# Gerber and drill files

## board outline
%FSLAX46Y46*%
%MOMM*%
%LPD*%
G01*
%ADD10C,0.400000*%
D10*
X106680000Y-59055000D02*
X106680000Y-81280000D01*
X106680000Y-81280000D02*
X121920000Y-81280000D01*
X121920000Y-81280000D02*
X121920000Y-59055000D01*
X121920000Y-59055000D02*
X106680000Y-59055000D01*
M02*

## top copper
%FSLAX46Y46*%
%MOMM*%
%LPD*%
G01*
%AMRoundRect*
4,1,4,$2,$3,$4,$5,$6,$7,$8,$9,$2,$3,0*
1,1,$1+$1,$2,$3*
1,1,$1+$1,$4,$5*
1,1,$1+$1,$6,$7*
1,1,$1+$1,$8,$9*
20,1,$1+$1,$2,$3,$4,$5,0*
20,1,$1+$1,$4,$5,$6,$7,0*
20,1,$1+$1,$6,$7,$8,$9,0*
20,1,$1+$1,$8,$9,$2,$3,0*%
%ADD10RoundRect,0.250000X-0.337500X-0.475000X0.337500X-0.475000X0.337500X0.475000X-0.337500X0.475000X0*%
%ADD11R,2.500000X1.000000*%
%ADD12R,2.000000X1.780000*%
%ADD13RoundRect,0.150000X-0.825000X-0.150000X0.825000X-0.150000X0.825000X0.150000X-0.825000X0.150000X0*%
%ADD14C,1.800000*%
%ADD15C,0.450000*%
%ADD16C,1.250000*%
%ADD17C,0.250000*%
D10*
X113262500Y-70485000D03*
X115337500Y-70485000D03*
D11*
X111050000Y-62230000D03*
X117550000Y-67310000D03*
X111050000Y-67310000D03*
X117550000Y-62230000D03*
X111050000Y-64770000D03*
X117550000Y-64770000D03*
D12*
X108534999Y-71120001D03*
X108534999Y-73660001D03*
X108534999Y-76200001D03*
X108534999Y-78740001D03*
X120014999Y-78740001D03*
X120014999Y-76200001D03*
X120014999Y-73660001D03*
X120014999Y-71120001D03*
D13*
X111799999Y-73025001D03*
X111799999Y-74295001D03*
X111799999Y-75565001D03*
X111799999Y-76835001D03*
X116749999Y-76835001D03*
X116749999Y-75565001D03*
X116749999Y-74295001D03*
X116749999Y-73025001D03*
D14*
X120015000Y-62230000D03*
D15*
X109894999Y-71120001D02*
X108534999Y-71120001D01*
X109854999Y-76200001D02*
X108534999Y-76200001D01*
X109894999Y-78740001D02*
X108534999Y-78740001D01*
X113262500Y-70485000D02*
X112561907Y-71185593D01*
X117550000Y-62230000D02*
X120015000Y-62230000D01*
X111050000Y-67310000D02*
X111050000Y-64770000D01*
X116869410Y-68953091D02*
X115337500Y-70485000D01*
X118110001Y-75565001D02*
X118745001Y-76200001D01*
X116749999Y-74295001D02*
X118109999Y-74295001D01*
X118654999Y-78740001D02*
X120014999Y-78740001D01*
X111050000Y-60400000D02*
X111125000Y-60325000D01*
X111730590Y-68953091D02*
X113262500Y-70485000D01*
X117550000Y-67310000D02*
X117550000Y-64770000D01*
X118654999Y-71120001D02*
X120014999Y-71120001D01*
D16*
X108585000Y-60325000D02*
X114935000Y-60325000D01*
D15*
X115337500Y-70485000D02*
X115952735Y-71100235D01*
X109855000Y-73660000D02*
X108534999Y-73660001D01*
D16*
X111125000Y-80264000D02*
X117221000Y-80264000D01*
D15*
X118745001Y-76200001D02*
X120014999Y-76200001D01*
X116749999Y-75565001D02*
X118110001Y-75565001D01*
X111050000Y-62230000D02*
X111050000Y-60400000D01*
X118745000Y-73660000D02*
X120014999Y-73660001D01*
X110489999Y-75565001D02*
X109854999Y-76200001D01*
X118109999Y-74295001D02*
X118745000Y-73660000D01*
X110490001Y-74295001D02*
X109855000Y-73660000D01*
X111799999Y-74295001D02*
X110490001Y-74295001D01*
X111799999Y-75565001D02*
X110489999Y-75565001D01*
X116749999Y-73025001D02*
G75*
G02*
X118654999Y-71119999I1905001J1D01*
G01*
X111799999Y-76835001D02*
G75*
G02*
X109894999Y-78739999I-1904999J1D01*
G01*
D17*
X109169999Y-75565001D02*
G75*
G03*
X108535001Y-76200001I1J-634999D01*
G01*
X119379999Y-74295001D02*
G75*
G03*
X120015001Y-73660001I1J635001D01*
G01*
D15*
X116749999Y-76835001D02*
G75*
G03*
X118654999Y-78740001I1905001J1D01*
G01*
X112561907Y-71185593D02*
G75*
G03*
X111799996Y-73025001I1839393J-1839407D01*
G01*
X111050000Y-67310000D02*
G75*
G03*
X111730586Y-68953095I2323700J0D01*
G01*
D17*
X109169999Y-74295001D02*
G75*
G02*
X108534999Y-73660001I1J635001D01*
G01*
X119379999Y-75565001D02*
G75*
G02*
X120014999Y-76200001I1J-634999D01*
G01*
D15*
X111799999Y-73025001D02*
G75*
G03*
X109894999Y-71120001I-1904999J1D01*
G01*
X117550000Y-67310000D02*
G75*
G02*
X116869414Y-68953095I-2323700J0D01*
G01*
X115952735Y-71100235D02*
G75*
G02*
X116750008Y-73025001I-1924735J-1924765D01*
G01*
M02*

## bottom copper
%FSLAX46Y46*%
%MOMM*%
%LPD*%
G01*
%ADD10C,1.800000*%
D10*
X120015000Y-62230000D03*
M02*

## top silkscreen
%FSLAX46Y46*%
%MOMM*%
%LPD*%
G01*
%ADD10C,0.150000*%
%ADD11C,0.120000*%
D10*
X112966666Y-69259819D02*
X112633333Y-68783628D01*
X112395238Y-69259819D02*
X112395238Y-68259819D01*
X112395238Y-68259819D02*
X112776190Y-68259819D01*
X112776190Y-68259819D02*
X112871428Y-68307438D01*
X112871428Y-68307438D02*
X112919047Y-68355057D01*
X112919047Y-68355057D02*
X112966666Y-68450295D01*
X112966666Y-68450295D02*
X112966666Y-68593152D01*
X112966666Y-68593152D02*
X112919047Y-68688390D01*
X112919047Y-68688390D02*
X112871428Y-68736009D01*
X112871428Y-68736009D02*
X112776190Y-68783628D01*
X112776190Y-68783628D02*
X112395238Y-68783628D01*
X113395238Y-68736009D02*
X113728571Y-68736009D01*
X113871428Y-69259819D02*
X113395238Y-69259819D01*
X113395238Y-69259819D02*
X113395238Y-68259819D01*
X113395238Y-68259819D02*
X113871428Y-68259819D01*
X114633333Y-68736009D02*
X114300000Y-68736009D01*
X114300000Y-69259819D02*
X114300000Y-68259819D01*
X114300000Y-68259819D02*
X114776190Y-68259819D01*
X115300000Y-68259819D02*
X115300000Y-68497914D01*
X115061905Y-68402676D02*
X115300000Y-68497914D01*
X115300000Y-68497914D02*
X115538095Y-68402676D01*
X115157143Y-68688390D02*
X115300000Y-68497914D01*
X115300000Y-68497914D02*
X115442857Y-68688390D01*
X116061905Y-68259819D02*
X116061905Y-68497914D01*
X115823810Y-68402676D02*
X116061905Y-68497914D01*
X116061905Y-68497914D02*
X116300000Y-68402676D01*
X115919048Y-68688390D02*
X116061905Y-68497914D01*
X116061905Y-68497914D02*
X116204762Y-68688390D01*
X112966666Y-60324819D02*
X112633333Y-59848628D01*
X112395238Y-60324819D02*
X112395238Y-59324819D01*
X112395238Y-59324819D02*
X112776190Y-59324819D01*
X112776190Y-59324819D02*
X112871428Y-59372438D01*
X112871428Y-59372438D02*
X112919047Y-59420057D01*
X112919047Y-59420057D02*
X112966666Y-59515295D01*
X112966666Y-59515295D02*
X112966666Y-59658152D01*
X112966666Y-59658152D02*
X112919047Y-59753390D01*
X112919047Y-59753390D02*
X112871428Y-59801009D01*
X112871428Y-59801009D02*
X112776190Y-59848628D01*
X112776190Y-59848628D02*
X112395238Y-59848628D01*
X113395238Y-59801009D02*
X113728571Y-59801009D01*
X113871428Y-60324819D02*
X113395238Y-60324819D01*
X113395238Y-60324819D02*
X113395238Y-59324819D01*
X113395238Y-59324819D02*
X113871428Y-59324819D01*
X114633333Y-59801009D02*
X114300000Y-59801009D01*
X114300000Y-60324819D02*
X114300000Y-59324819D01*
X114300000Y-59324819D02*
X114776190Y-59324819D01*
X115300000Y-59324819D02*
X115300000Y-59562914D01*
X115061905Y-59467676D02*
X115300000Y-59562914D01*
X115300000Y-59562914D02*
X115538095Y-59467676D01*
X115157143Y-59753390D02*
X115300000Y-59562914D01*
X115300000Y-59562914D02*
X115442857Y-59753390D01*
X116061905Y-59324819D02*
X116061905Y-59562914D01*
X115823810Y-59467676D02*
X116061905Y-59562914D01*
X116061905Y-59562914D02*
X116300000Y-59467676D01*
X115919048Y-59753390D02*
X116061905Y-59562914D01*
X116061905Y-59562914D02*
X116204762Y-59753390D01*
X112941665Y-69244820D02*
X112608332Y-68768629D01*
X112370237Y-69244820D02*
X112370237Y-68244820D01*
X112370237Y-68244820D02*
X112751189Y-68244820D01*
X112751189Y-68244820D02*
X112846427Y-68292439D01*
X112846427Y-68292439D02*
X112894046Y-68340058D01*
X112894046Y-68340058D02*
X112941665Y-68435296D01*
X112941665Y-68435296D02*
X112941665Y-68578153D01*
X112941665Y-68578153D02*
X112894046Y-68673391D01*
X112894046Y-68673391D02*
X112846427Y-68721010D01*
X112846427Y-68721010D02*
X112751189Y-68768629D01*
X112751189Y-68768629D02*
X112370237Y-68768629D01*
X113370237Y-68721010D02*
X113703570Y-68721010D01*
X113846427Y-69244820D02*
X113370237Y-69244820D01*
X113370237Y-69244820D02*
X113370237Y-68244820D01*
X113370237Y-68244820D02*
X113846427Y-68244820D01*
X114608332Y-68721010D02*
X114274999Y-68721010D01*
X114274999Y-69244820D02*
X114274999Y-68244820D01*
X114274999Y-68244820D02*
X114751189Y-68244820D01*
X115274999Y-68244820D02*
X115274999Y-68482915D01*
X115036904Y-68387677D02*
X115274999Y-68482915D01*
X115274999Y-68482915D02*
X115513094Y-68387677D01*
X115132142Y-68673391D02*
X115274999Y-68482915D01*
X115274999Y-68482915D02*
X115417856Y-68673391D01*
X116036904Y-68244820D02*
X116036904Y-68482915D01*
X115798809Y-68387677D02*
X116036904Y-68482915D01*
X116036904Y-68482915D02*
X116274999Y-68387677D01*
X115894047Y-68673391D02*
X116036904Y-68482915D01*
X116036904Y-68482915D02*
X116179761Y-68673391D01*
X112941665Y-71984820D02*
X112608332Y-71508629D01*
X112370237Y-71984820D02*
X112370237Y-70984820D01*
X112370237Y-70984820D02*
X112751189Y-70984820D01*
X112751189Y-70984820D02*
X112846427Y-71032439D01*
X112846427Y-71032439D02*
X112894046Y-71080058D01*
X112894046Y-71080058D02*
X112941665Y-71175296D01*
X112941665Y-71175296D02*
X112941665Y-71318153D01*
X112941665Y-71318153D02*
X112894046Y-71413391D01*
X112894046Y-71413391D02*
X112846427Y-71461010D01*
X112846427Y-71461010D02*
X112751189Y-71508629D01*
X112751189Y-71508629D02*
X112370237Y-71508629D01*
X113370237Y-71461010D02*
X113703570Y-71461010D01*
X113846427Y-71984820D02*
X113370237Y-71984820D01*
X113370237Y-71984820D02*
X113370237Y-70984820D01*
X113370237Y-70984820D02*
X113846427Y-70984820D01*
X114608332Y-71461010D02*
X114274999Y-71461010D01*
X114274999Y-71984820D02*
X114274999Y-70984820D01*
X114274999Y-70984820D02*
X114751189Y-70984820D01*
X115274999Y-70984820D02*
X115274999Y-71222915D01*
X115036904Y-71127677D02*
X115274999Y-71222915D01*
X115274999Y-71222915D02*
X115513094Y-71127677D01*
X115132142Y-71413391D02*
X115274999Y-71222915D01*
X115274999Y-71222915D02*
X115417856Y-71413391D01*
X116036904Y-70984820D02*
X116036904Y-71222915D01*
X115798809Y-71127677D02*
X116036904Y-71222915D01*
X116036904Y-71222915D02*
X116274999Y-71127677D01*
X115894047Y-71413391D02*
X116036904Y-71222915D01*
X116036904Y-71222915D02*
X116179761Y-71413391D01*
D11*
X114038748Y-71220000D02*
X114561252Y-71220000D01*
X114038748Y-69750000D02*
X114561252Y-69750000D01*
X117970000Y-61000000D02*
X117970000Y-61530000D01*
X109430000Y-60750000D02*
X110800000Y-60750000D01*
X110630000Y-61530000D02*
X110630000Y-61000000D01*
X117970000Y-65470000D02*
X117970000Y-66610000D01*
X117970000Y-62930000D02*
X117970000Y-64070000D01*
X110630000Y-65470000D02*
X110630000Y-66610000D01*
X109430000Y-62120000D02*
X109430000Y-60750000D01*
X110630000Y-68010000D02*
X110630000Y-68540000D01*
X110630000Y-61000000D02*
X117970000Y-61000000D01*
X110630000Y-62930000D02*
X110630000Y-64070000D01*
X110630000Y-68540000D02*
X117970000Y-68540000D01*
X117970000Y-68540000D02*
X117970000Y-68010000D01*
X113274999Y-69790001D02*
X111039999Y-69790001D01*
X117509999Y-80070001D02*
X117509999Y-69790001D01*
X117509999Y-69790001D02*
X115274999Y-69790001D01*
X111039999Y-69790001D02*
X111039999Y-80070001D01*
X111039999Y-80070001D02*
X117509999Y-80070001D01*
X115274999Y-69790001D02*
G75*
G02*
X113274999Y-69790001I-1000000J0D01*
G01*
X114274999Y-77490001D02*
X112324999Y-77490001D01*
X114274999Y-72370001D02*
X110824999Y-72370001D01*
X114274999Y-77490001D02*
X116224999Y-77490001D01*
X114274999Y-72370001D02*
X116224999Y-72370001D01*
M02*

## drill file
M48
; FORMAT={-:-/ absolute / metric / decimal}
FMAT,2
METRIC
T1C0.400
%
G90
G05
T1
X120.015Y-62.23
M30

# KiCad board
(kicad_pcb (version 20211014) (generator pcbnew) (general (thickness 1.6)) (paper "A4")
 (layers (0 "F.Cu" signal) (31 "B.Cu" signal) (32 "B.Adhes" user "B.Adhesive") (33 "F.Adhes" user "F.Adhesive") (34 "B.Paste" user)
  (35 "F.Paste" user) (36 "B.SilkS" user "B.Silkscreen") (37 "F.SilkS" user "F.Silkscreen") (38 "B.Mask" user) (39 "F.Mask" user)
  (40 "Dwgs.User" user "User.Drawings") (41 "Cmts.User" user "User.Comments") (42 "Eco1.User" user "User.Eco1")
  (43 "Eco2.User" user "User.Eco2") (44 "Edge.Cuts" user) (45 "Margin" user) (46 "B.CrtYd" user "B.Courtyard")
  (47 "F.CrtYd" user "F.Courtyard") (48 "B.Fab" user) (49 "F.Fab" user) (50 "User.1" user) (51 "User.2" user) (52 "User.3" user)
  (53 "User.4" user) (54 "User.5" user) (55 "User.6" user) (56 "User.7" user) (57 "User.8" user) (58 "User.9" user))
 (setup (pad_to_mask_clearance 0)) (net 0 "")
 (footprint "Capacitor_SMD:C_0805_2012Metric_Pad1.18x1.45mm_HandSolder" (layer "F.Cu") (at 114.3 70.485)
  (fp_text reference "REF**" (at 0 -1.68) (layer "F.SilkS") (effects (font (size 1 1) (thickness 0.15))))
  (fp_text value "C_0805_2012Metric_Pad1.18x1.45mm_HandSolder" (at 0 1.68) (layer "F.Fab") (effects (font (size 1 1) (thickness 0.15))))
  (fp_line (start -0.261252 0.735) (end 0.261252 0.735) (layer "F.SilkS") (width 0.12))
  (fp_line (start -0.261252 -0.735) (end 0.261252 -0.735) (layer "F.SilkS") (width 0.12))
  (pad "1" smd roundrect (at -1.0375 0) (size 1.175 1.45) (layers "F.Cu" "F.Paste" "F.Mask") (roundrect_rratio 0.2127659574))
  (pad "2" smd roundrect (at 1.0375 0) (size 1.175 1.45) (layers "F.Cu" "F.Paste" "F.Mask") (roundrect_rratio 0.2127659574)))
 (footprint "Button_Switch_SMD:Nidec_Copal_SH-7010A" (layer "F.Cu") (at 114.3 64.77)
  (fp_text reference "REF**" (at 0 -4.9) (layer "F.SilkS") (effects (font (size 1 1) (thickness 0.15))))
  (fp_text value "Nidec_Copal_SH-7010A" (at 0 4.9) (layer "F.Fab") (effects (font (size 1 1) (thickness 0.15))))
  (fp_line (start 3.67 -3.77) (end 3.67 -3.24) (layer "F.SilkS") (width 0.12))
  (fp_line (start -4.87 -4.02) (end -3.5 -4.02) (layer "F.SilkS") (width 0.12))
  (fp_line (start -3.67 -3.24) (end -3.67 -3.77) (layer "F.SilkS") (width 0.12))
  (fp_line (start 3.67 0.7) (end 3.67 1.84) (layer "F.SilkS") (width 0.12))
  (fp_line (start 3.67 -1.84) (end 3.67 -0.7) (layer "F.SilkS") (width 0.12))
  (fp_line (start -3.67 0.7) (end -3.67 1.84) (layer "F.SilkS") (width 0.12))
  (fp_line (start -4.87 -2.65) (end -4.87 -4.02) (layer "F.SilkS") (width 0.12))
  (fp_line (start -3.67 3.24) (end -3.67 3.77) (layer "F.SilkS") (width 0.12))
  (fp_line (start -3.67 -3.77) (end 3.67 -3.77) (layer "F.SilkS") (width 0.12))
  (fp_line (start -3.67 -1.84) (end -3.67 -0.7) (layer "F.SilkS") (width 0.12))
  (fp_line (start -3.67 3.77) (end 3.67 3.77) (layer "F.SilkS") (width 0.12))
  (fp_line (start 3.67 3.77) (end 3.67 3.24) (layer "F.SilkS") (width 0.12))
  (pad "1" smd rect (at -3.25 -2.54) (size 2.5 1) (layers "F.Cu" "F.Paste" "F.Mask"))
  (pad "2" smd rect (at 3.25 2.54) (size 2.5 1) (layers "F.Cu" "F.Paste" "F.Mask"))
  (pad "4" smd rect (at -3.25 2.54) (size 2.5 1) (layers "F.Cu" "F.Paste" "F.Mask"))
  (pad "8" smd rect (at 3.25 -2.54) (size 2.5 1) (layers "F.Cu" "F.Paste" "F.Mask"))
  (pad "C" smd rect (at -3.25 0) (size 2.5 1) (layers "F.Cu" "F.Paste" "F.Mask"))
  (pad "C" smd rect (at 3.25 0) (size 2.5 1) (layers "F.Cu" "F.Paste" "F.Mask")))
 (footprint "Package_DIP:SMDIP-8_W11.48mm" (layer "F.Cu") (at 114.274999 74.930001)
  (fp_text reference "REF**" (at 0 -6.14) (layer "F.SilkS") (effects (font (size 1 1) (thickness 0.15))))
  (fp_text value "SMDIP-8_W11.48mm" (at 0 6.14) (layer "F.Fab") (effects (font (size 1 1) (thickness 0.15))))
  (fp_line (start -1 -5.14) (end -3.235 -5.14) (layer "F.SilkS") (width 0.12))
  (fp_line (start 3.235 5.14) (end 3.235 -5.14) (layer "F.SilkS") (width 0.12))
  (fp_line (start 3.235 -5.14) (end 1 -5.14) (layer "F.SilkS") (width 0.12))
  (fp_line (start -3.235 -5.14) (end -3.235 5.14) (layer "F.SilkS") (width 0.12))
  (fp_line (start -3.235 5.14) (end 3.235 5.14) (layer "F.SilkS") (width 0.12))
  (fp_arc (start 1 -5.14) (mid 0 -4.14) (end -1 -5.14) (layer "F.SilkS") (width 0.12))
  (pad "1" smd rect (at -5.74 -3.81) (size 2 1.78) (layers "F.Cu" "F.Paste" "F.Mask"))
  (pad "2" smd rect (at -5.74 -1.27) (size 2 1.78) (layers "F.Cu" "F.Paste" "F.Mask"))
  (pad "3" smd rect (at -5.74 1.27) (size 2 1.78) (layers "F.Cu" "F.Paste" "F.Mask"))
  (pad "4" smd rect (at -5.74 3.81) (size 2 1.78) (layers "F.Cu" "F.Paste" "F.Mask"))
  (pad "5" smd rect (at 5.74 3.81) (size 2 1.78) (layers "F.Cu" "F.Paste" "F.Mask"))
  (pad "6" smd rect (at 5.74 1.27) (size 2 1.78) (layers "F.Cu" "F.Paste" "F.Mask"))
  (pad "7" smd rect (at 5.74 -1.27) (size 2 1.78) (layers "F.Cu" "F.Paste" "F.Mask"))
  (pad "8" smd rect (at 5.74 -3.81) (size 2 1.78) (layers "F.Cu" "F.Paste" "F.Mask")))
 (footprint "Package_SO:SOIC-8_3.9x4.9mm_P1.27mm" (layer "F.Cu") (at 114.274999 74.930001)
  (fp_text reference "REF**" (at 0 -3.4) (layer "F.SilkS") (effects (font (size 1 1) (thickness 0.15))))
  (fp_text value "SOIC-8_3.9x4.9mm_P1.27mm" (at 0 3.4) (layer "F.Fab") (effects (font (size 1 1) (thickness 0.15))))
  (fp_line (start 0 2.56) (end -1.95 2.56) (layer "F.SilkS") (width 0.12))
  (fp_line (start 0 -2.56) (end -3.45 -2.56) (layer "F.SilkS") (width 0.12))
  (fp_line (start 0 2.56) (end 1.95 2.56) (layer "F.SilkS") (width 0.12))
  (fp_line (start 0 -2.56) (end 1.95 -2.56) (layer "F.SilkS") (width 0.12))
  (pad "1" smd roundrect (at -2.475 -1.905) (size 1.95 0.6) (layers "F.Cu" "F.Paste" "F.Mask") (roundrect_rratio 0.25))
  (pad "2" smd roundrect (at -2.475 -0.635) (size 1.95 0.6) (layers "F.Cu" "F.Paste" "F.Mask") (roundrect_rratio 0.25))
  (pad "3" smd roundrect (at -2.475 0.635) (size 1.95 0.6) (layers "F.Cu" "F.Paste" "F.Mask") (roundrect_rratio 0.25))
  (pad "4" smd roundrect (at -2.475 1.905) (size 1.95 0.6) (layers "F.Cu" "F.Paste" "F.Mask") (roundrect_rratio 0.25))
  (pad "5" smd roundrect (at 2.475 1.905) (size 1.95 0.6) (layers "F.Cu" "F.Paste" "F.Mask") (roundrect_rratio 0.25))
  (pad "6" smd roundrect (at 2.475 0.635) (size 1.95 0.6) (layers "F.Cu" "F.Paste" "F.Mask") (roundrect_rratio 0.25))
  (pad "7" smd roundrect (at 2.475 -0.635) (size 1.95 0.6) (layers "F.Cu" "F.Paste" "F.Mask") (roundrect_rratio 0.25))
  (pad "8" smd roundrect (at 2.475 -1.905) (size 1.95 0.6) (layers "F.Cu" "F.Paste" "F.Mask") (roundrect_rratio 0.25)))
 (gr_line (start 106.68 59.055) (end 106.68 81.28) (layer "Edge.Cuts") (width 0.4))
 (gr_line (start 106.68 81.28) (end 121.92 81.28) (layer "Edge.Cuts") (width 0.4))
 (gr_line (start 121.92 81.28) (end 121.92 59.055) (layer "Edge.Cuts") (width 0.4))
 (gr_line (start 121.92 59.055) (end 106.68 59.055) (layer "Edge.Cuts") (width 0.4))
 (segment (start 109.894999 71.120001) (end 108.534999 71.120001) (width 0.45) (layer "F.Cu") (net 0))
 (segment (start 109.854999 76.200001) (end 108.534999 76.200001) (width 0.45) (layer "F.Cu") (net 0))
 (segment (start 109.894999 78.740001) (end 108.534999 78.740001) (width 0.45) (layer "F.Cu") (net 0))
 (segment (start 113.2625 70.485) (end 112.561907 71.185593) (width 0.45) (layer "F.Cu") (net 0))
 (segment (start 117.55 62.23) (end 120.015 62.23) (width 0.45) (layer "F.Cu") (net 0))
 (segment (start 111.05 67.31) (end 111.05 64.77) (width 0.45) (layer "F.Cu") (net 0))
 (segment (start 116.86941 68.953091) (end 115.3375 70.485) (width 0.45) (layer "F.Cu") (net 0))
 (segment (start 118.110001 75.565001) (end 118.745001 76.200001) (width 0.45) (layer "F.Cu") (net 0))
 (segment (start 116.749999 74.295001) (end 118.109999 74.295001) (width 0.45) (layer "F.Cu") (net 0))
 (segment (start 118.654999 78.740001) (end 120.014999 78.740001) (width 0.45) (layer "F.Cu") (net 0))
 (segment (start 111.05 60.4) (end 111.125 60.325) (width 0.45) (layer "F.Cu") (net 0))
 (segment (start 111.73059 68.953091) (end 113.2625 70.485) (width 0.45) (layer "F.Cu") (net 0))
 (segment (start 117.55 67.31) (end 117.55 64.77) (width 0.45) (layer "F.Cu") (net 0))
 (segment (start 118.654999 71.120001) (end 120.014999 71.120001) (width 0.45) (layer "F.Cu") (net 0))
 (segment (start 108.585 60.325) (end 114.935 60.325) (width 1.25) (layer "F.Cu") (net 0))
 (segment (start 115.3375 70.485) (end 115.952735 71.100235) (width 0.45) (layer "F.Cu") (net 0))
 (segment (start 109.855 73.66) (end 108.534999 73.660001) (width 0.45) (layer "F.Cu") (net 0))
 (segment (start 111.125 80.264) (end 117.221 80.264) (width 1.25) (layer "F.Cu") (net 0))
 (segment (start 118.745001 76.200001) (end 120.014999 76.200001) (width 0.45) (layer "F.Cu") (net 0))
 (segment (start 116.749999 75.565001) (end 118.110001 75.565001) (width 0.45) (layer "F.Cu") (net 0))
 (segment (start 111.05 62.23) (end 111.05 60.4) (width 0.45) (layer "F.Cu") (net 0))
 (segment (start 118.745 73.66) (end 120.014999 73.660001) (width 0.45) (layer "F.Cu") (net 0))
 (segment (start 110.489999 75.565001) (end 109.854999 76.200001) (width 0.45) (layer "F.Cu") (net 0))
 (segment (start 118.109999 74.295001) (end 118.745 73.66) (width 0.45) (layer "F.Cu") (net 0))
 (segment (start 110.490001 74.295001) (end 109.855 73.66) (width 0.45) (layer "F.Cu") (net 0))
 (segment (start 111.799999 74.295001) (end 110.490001 74.295001) (width 0.45) (layer "F.Cu") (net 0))
 (segment (start 111.799999 75.565001) (end 110.489999 75.565001) (width 0.45) (layer "F.Cu") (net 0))
 (via (at 120.015 62.23) (size 1.8) (drill 0.4) (layers "F.Cu" "B.Cu") (free) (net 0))
 (arc (start 116.749999 73.025001) (mid 117.307961 71.677963) (end 118.654999 71.120001) (width 0.45) (layer "F.Cu") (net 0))
 (arc (start 111.799999 76.835001) (mid 111.242037 78.182039) (end 109.894999 78.740001) (width 0.45) (layer "F.Cu") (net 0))
 (arc (start 109.169999 75.565001) (mid 108.720986 75.750988) (end 108.534999 76.200001) (width 0.25) (layer "F.Cu") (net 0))
 (arc (start 119.379999 74.295001) (mid 119.829012 74.109014) (end 120.014999 73.660001) (width 0.25) (layer "F.Cu") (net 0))
 (arc (start 116.749999 76.835001) (mid 117.307961 78.182039) (end 118.654999 78.740001) (width 0.45) (layer "F.Cu") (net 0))
 (arc (start 112.561907 71.185593) (mid 111.998013 72.02952) (end 111.799999 73.025001) (width 0.45) (layer "F.Cu") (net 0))
 (arc (start 111.05 67.31) (mid 111.22688 68.199234) (end 111.73059 68.953091) (width 0.45) (layer "F.Cu") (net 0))
 (arc (start 109.169999 74.295001) (mid 108.720986 74.109014) (end 108.534999 73.660001) (width 0.25) (layer "F.Cu") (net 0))
 (arc (start 119.379999 75.565001) (mid 119.829012 75.750988) (end 120.014999 76.200001) (width 0.25) (layer "F.Cu") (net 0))
 (arc (start 111.799999 73.025001) (mid 111.242037 71.677963) (end 109.894999 71.120001) (width 0.45) (layer "F.Cu") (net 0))
 (arc (start 117.55 67.31) (mid 117.37312 68.199234) (end 116.86941 68.953091) (width 0.45) (layer "F.Cu") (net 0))
 (arc (start 115.952735 71.100235) (mid 116.542797 71.983325) (end 116.749999 73.025001) (width 0.45) (layer "F.Cu") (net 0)))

